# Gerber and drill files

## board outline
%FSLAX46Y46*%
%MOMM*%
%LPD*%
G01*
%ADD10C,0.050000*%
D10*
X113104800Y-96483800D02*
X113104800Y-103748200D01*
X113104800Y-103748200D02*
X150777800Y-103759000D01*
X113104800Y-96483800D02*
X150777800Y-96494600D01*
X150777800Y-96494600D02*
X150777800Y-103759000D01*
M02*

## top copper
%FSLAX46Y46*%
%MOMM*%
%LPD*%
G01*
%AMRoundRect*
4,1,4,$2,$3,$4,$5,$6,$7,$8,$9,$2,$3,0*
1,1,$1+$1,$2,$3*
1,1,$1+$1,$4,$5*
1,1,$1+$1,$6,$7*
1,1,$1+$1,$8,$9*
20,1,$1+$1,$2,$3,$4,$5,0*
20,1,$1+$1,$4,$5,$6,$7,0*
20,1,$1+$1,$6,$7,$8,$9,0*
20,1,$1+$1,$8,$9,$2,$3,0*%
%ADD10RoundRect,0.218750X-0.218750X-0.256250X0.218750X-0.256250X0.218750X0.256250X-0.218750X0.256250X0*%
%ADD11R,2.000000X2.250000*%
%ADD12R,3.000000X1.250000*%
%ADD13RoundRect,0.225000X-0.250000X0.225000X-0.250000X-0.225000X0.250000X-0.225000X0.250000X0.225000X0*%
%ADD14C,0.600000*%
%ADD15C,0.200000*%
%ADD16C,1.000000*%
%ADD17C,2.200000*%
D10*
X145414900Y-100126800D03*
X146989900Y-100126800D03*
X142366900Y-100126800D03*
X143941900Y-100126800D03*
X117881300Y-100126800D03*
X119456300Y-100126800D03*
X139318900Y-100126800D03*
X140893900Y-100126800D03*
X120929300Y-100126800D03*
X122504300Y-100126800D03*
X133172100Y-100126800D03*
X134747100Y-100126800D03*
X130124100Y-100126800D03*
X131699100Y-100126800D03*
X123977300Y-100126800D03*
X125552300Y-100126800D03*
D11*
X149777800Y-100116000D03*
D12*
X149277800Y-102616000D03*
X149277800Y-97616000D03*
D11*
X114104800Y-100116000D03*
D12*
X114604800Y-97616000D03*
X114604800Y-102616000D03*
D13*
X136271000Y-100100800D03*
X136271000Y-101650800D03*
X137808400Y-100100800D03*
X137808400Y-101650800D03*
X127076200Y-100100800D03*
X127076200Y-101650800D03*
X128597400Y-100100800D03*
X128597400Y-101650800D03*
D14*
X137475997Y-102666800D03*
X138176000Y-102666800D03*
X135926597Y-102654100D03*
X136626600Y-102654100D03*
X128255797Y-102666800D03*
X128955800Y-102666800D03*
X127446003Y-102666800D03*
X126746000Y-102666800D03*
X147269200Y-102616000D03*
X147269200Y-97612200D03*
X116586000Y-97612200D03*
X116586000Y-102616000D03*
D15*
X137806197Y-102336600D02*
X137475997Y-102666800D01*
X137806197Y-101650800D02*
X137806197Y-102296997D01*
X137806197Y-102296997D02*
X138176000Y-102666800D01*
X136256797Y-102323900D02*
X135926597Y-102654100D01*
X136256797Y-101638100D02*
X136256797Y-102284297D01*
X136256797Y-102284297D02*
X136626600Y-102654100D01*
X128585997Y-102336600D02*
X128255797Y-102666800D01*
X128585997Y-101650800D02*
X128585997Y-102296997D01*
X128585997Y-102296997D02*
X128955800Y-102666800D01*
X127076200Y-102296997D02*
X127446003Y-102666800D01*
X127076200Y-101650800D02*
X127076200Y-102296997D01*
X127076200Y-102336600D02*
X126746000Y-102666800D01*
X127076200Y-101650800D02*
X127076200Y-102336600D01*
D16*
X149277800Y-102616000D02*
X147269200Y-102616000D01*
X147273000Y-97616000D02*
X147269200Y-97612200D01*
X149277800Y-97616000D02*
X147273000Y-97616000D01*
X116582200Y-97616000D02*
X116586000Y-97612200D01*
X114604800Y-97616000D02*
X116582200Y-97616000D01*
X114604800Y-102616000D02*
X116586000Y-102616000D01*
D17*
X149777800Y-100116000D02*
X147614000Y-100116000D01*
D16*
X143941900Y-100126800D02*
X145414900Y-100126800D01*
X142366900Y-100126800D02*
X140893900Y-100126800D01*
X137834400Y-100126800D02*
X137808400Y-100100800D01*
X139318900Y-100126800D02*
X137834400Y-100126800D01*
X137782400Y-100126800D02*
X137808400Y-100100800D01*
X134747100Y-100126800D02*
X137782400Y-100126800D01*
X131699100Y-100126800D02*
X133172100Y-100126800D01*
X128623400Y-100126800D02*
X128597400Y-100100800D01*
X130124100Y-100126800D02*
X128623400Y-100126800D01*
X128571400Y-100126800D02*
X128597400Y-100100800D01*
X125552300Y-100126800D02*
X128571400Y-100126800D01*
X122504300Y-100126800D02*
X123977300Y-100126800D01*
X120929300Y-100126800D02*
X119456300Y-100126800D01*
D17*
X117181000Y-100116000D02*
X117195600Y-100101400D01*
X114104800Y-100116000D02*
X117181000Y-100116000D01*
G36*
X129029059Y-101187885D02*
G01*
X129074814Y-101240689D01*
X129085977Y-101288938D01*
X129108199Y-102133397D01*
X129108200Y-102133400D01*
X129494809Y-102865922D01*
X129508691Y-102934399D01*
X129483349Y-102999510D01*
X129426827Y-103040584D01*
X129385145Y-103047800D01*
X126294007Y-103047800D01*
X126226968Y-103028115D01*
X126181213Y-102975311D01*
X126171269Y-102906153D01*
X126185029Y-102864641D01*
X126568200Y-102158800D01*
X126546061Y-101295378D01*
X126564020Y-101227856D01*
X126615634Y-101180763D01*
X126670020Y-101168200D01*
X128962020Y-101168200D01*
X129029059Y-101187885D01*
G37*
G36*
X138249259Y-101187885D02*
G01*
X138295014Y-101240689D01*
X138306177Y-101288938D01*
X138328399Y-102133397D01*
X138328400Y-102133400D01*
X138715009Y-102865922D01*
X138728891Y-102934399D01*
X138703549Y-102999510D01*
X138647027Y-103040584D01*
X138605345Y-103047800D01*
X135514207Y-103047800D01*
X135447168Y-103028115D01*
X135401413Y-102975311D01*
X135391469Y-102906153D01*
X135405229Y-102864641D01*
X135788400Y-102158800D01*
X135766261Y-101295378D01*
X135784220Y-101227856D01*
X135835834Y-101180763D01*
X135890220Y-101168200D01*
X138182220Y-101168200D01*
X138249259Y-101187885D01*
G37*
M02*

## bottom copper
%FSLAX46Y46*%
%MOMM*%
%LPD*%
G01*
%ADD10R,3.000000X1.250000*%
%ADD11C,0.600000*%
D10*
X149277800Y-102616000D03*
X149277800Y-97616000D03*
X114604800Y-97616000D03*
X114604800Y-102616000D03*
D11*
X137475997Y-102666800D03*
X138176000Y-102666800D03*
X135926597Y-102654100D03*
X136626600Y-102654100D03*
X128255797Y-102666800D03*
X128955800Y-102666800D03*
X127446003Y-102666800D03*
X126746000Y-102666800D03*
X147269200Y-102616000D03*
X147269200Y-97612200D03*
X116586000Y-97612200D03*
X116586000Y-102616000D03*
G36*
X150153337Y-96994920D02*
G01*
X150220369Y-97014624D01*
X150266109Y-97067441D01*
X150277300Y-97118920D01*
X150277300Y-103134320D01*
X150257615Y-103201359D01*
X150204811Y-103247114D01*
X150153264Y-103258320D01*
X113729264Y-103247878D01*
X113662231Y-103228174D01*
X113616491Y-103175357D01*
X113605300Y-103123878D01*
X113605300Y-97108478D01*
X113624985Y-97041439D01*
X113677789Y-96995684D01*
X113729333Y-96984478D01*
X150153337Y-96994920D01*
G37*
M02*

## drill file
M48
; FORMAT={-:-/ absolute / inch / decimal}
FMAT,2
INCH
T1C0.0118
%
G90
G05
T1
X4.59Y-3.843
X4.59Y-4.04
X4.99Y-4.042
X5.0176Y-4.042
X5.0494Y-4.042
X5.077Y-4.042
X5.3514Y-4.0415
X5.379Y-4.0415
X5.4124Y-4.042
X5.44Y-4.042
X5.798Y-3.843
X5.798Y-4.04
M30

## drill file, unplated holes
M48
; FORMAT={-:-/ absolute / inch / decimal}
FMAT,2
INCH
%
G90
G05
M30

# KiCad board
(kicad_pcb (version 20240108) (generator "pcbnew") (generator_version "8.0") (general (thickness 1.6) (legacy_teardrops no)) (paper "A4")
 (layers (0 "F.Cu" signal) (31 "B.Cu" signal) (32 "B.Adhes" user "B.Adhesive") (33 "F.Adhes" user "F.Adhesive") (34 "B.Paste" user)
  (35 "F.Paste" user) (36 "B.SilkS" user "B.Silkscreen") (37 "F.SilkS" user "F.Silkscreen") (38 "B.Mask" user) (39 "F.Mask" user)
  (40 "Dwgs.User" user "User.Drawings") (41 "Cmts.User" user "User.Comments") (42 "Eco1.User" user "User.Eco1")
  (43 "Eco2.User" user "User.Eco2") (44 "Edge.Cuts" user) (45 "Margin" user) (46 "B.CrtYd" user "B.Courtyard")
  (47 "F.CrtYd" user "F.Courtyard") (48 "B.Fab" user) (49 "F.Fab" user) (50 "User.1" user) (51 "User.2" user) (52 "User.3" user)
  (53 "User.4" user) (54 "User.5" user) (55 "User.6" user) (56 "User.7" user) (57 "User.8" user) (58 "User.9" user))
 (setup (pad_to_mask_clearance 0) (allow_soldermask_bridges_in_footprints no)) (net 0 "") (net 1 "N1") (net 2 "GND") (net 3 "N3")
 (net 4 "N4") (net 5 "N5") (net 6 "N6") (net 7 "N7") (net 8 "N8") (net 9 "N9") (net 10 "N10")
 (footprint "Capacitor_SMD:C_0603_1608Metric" (layer "F.Cu") (at 128.5974 100.8758 -90)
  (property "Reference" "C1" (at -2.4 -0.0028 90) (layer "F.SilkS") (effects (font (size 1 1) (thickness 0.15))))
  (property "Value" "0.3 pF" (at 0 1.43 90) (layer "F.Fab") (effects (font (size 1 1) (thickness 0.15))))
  (pad "1" smd roundrect (at -0.775 0 270) (size 0.9 0.95) (layers "F.Cu" "F.Paste" "F.Mask") (roundrect_rratio 0.25) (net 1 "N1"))
  (pad "2" smd roundrect (at 0.775 0 270) (size 0.9 0.95) (layers "F.Cu" "F.Paste" "F.Mask") (roundrect_rratio 0.25) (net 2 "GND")))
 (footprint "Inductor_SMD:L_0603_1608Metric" (layer "F.Cu") (at 133.9596 100.1268)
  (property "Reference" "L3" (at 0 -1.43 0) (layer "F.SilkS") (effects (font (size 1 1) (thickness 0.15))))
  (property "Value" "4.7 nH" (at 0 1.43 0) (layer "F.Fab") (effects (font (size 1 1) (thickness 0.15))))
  (pad "1" smd roundrect (at -0.7875 0) (size 0.875 0.95) (layers "F.Cu" "F.Paste" "F.Mask") (roundrect_rratio 0.25) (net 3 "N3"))
  (pad "2" smd roundrect (at 0.7875 0) (size 0.875 0.95) (layers "F.Cu" "F.Paste" "F.Mask") (roundrect_rratio 0.25) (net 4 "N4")))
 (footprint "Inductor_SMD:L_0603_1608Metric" (layer "F.Cu") (at 146.2024 100.1268)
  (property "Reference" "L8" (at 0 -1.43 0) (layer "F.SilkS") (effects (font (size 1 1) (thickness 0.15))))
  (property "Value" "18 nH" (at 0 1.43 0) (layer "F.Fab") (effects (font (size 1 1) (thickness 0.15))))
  (pad "1" smd roundrect (at -0.7875 0) (size 0.875 0.95) (layers "F.Cu" "F.Paste" "F.Mask") (roundrect_rratio 0.25) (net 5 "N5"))
  (pad "2" smd roundrect (at 0.7875 0) (size 0.875 0.95) (layers "F.Cu" "F.Paste" "F.Mask") (roundrect_rratio 0.25) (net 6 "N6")))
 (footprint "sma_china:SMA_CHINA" (layer "F.Cu") (at 150.7778 100.116 90)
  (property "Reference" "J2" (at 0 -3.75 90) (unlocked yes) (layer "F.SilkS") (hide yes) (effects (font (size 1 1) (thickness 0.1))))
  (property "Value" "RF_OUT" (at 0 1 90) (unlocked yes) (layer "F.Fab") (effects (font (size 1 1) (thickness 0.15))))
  (pad "1" smd rect (at 0 -1 90) (size 2.25 2) (layers "F.Cu" "F.Paste" "F.Mask") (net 6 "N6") (thermal_bridge_angle 45))
  (pad "2" smd rect (at -2.5 -1.5 90) (size 1.25 3) (layers "F.Cu" "F.Paste" "F.Mask") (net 2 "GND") (thermal_bridge_angle 45))
  (pad "2" smd rect (at -2.5 -1.5 90) (size 1.25 3) (layers "B.Cu" "B.Paste" "B.Mask") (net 2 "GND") (thermal_bridge_angle 45))
  (pad "2" smd rect (at 2.5 -1.5 90) (size 1.25 3) (layers "F.Cu" "F.Paste" "F.Mask") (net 2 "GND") (thermal_bridge_angle 45))
  (pad "2" smd rect (at 2.5 -1.5 90) (size 1.25 3) (layers "B.Cu" "B.Paste" "B.Mask") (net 2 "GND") (thermal_bridge_angle 45)))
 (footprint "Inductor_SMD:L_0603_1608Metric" (layer "F.Cu") (at 121.7168 100.1268)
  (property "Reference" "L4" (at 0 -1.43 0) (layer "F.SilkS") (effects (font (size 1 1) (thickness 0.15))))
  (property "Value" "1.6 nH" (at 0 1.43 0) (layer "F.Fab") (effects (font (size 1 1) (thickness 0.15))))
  (pad "1" smd roundrect (at -0.7875 0) (size 0.875 0.95) (layers "F.Cu" "F.Paste" "F.Mask") (roundrect_rratio 0.25) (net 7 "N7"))
  (pad "2" smd roundrect (at 0.7875 0) (size 0.875 0.95) (layers "F.Cu" "F.Paste" "F.Mask") (roundrect_rratio 0.25) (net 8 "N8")))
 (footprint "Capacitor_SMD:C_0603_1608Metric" (layer "F.Cu") (at 137.8084 100.8758 -90)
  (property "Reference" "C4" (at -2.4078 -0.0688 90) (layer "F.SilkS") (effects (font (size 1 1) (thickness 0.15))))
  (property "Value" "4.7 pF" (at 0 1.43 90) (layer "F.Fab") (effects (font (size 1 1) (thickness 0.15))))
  (pad "1" smd roundrect (at -0.775 0 270) (size 0.9 0.95) (layers "F.Cu" "F.Paste" "F.Mask") (roundrect_rratio 0.25) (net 4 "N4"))
  (pad "2" smd roundrect (at 0.775 0 270) (size 0.9 0.95) (layers "F.Cu" "F.Paste" "F.Mask") (roundrect_rratio 0.25) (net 2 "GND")))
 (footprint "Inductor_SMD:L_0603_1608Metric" (layer "F.Cu") (at 124.7648 100.1268)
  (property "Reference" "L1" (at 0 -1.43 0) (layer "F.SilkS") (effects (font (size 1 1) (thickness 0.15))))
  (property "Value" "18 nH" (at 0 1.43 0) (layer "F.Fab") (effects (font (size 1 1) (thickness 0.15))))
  (pad "1" smd roundrect (at -0.7875 0) (size 0.875 0.95) (layers "F.Cu" "F.Paste" "F.Mask") (roundrect_rratio 0.25) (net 8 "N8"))
  (pad "2" smd roundrect (at 0.7875 0) (size 0.875 0.95) (layers "F.Cu" "F.Paste" "F.Mask") (roundrect_rratio 0.25) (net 1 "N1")))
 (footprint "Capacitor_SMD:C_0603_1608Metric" (layer "F.Cu") (at 127.0762 100.8758 -90)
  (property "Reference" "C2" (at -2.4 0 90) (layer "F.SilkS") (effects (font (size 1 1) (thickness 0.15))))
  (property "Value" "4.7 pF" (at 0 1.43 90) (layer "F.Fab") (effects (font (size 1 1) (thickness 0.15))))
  (pad "1" smd roundrect (at -0.775 0 270) (size 0.9 0.95) (layers "F.Cu" "F.Paste" "F.Mask") (roundrect_rratio 0.25) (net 1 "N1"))
  (pad "2" smd roundrect (at 0.775 0 270) (size 0.9 0.95) (layers "F.Cu" "F.Paste" "F.Mask") (roundrect_rratio 0.25) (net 2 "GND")))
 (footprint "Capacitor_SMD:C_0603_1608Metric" (layer "F.Cu") (at 136.271 100.8758 -90)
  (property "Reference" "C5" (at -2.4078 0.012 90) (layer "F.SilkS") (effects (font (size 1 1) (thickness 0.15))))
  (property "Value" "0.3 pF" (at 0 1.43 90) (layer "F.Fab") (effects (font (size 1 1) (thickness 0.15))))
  (pad "1" smd roundrect (at -0.775 0 270) (size 0.9 0.95) (layers "F.Cu" "F.Paste" "F.Mask") (roundrect_rratio 0.25) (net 4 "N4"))
  (pad "2" smd roundrect (at 0.775 0 270) (size 0.9 0.95) (layers "F.Cu" "F.Paste" "F.Mask") (roundrect_rratio 0.25) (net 2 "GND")))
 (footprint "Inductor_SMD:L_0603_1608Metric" (layer "F.Cu") (at 130.9116 100.1268)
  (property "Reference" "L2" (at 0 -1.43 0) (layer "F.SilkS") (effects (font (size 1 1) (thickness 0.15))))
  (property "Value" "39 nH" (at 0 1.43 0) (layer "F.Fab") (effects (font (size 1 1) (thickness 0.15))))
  (pad "1" smd roundrect (at -0.7875 0) (size 0.875 0.95) (layers "F.Cu" "F.Paste" "F.Mask") (roundrect_rratio 0.25) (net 1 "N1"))
  (pad "2" smd roundrect (at 0.7875 0) (size 0.875 0.95) (layers "F.Cu" "F.Paste" "F.Mask") (roundrect_rratio 0.25) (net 3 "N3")))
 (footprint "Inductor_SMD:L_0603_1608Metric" (layer "F.Cu") (at 140.1064 100.1268)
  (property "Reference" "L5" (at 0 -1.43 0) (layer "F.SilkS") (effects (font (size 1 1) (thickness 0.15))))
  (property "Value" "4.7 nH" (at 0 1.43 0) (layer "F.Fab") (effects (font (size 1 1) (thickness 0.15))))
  (pad "1" smd roundrect (at -0.7875 0) (size 0.875 0.95) (layers "F.Cu" "F.Paste" "F.Mask") (roundrect_rratio 0.25) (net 4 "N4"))
  (pad "2" smd roundrect (at 0.7875 0) (size 0.875 0.95) (layers "F.Cu" "F.Paste" "F.Mask") (roundrect_rratio 0.25) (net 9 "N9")))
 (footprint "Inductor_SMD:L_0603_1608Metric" (layer "F.Cu") (at 143.1544 100.1268)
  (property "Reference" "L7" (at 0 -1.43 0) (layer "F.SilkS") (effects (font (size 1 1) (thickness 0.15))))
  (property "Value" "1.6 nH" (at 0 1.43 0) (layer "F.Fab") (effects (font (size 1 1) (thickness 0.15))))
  (pad "1" smd roundrect (at -0.7875 0) (size 0.875 0.95) (layers "F.Cu" "F.Paste" "F.Mask") (roundrect_rratio 0.25) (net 9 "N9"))
  (pad "2" smd roundrect (at 0.7875 0) (size 0.875 0.95) (layers "F.Cu" "F.Paste" "F.Mask") (roundrect_rratio 0.25) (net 5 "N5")))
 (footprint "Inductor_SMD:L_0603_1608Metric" (layer "F.Cu") (at 118.6688 100.1268)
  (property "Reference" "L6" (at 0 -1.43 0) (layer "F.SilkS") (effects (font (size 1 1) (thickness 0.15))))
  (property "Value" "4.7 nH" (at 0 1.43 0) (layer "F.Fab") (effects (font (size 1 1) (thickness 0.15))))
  (pad "1" smd roundrect (at -0.7875 0) (size 0.875 0.95) (layers "F.Cu" "F.Paste" "F.Mask") (roundrect_rratio 0.25) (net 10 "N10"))
  (pad "2" smd roundrect (at 0.7875 0) (size 0.875 0.95) (layers "F.Cu" "F.Paste" "F.Mask") (roundrect_rratio 0.25) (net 7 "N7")))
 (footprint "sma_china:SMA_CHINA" (layer "F.Cu") (at 113.1048 100.116 -90)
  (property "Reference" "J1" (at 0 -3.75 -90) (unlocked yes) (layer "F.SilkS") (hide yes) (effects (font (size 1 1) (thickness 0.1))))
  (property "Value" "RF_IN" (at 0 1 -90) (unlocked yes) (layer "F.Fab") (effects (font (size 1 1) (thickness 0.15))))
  (pad "1" smd rect (at 0 -1 270) (size 2.25 2) (layers "F.Cu" "F.Paste" "F.Mask") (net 10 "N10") (thermal_bridge_angle 45))
  (pad "2" smd rect (at -2.5 -1.5 270) (size 1.25 3) (layers "F.Cu" "F.Paste" "F.Mask") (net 2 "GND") (thermal_bridge_angle 45))
  (pad "2" smd rect (at -2.5 -1.5 270) (size 1.25 3) (layers "B.Cu" "B.Paste" "B.Mask") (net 2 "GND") (thermal_bridge_angle 45))
  (pad "2" smd rect (at 2.5 -1.5 270) (size 1.25 3) (layers "F.Cu" "F.Paste" "F.Mask") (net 2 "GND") (thermal_bridge_angle 45))
  (pad "2" smd rect (at 2.5 -1.5 270) (size 1.25 3) (layers "B.Cu" "B.Paste" "B.Mask") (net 2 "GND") (thermal_bridge_angle 45)))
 (gr_line (start 150.7778 96.4946) (end 150.7778 103.759) (stroke (width 0.05) (type default)) (layer "Edge.Cuts"))
 (gr_line (start 113.1048 96.4838) (end 150.7778 96.4946) (stroke (width 0.05) (type default)) (layer "Edge.Cuts"))
 (gr_line (start 113.1048 96.4838) (end 113.1048 103.7482) (stroke (width 0.05) (type default)) (layer "Edge.Cuts"))
 (gr_line (start 113.1048 103.7482) (end 150.7778 103.759) (stroke (width 0.05) (type default)) (layer "Edge.Cuts"))
 (segment (start 147.273 97.616) (end 147.2692 97.6122) (width 1) (layer "F.Cu") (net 2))
 (segment (start 136.256797 101.6381) (end 136.256797 102.284297) (width 0.2) (layer "F.Cu") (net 2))
 (segment (start 127.0762 102.296997) (end 127.446003 102.6668) (width 0.2) (layer "F.Cu") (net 2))
 (segment (start 137.806197 101.6508) (end 137.806197 102.296997) (width 0.2) (layer "F.Cu") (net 2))
 (segment (start 127.0762 101.6508) (end 127.0762 102.296997) (width 0.2) (layer "F.Cu") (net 2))
 (segment (start 137.806197 102.3366) (end 137.475997 102.6668) (width 0.2) (layer "F.Cu") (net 2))
 (segment (start 127.0762 101.6508) (end 127.0762 102.3366) (width 0.2) (layer "F.Cu") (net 2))
 (segment (start 114.6048 102.616) (end 116.586 102.616) (width 1) (layer "F.Cu") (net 2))
 (segment (start 149.2778 97.616) (end 147.273 97.616) (width 1) (layer "F.Cu") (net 2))
 (segment (start 128.585997 101.6508) (end 128.585997 102.296997) (width 0.2) (layer "F.Cu") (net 2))
 (segment (start 128.585997 102.3366) (end 128.255797 102.6668) (width 0.2) (layer "F.Cu") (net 2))
 (segment (start 127.0762 102.3366) (end 126.746 102.6668) (width 0.2) (layer "F.Cu") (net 2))
 (segment (start 149.2778 102.616) (end 147.2692 102.616) (width 1) (layer "F.Cu") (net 2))
 (segment (start 136.256797 102.284297) (end 136.6266 102.6541) (width 0.2) (layer "F.Cu") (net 2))
 (segment (start 128.585997 102.296997) (end 128.9558 102.6668) (width 0.2) (layer "F.Cu") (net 2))
 (segment (start 136.256797 102.3239) (end 135.926597 102.6541) (width 0.2) (layer "F.Cu") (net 2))
 (segment (start 137.806197 102.296997) (end 138.176 102.6668) (width 0.2) (layer "F.Cu") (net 2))
 (segment (start 114.6048 97.616) (end 116.5822 97.616) (width 1) (layer "F.Cu") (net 2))
 (segment (start 116.5822 97.616) (end 116.586 97.6122) (width 1) (layer "F.Cu") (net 2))
 (via (at 136.6266 102.6541) (size 0.6) (drill 0.3) (layers "F.Cu" "B.Cu") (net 2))
 (via (at 138.176 102.6668) (size 0.6) (drill 0.3) (layers "F.Cu" "B.Cu") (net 2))
 (via (at 135.926597 102.6541) (size 0.6) (drill 0.3) (layers "F.Cu" "B.Cu") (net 2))
 (via (at 126.746 102.6668) (size 0.6) (drill 0.3) (layers "F.Cu" "B.Cu") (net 2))
 (via (at 137.475997 102.6668) (size 0.6) (drill 0.3) (layers "F.Cu" "B.Cu") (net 2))
 (via (at 127.446003 102.6668) (size 0.6) (drill 0.3) (layers "F.Cu" "B.Cu") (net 2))
 (via (at 116.586 102.616) (size 0.6) (drill 0.3) (layers "F.Cu" "B.Cu") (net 2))
 (via (at 128.255797 102.6668) (size 0.6) (drill 0.3) (layers "F.Cu" "B.Cu") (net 2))
 (via (at 116.586 97.6122) (size 0.6) (drill 0.3) (layers "F.Cu" "B.Cu") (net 2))
 (via (at 128.9558 102.6668) (size 0.6) (drill 0.3) (layers "F.Cu" "B.Cu") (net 2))
 (via (at 147.2692 97.6122) (size 0.6) (drill 0.3) (layers "F.Cu" "B.Cu") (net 2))
 (via (at 147.2692 102.616) (size 0.6) (drill 0.3) (layers "F.Cu" "B.Cu") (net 2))
 (segment (start 128.6234 100.1268) (end 128.5974 100.1008) (width 1) (layer "F.Cu") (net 1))
 (segment (start 130.1241 100.1268) (end 128.6234 100.1268) (width 1) (layer "F.Cu") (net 1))
 (segment (start 125.5523 100.1268) (end 128.5714 100.1268) (width 1) (layer "F.Cu") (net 1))
 (segment (start 128.5714 100.1268) (end 128.5974 100.1008) (width 1) (layer "F.Cu") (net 1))
 (segment (start 134.7471 100.1268) (end 137.7824 100.1268) (width 1) (layer "F.Cu") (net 4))
 (segment (start 137.7824 100.1268) (end 137.8084 100.1008) (width 1) (layer "F.Cu") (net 4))
 (segment (start 137.8344 100.1268) (end 137.8084 100.1008) (width 1) (layer "F.Cu") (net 4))
 (segment (start 139.3189 100.1268) (end 137.8344 100.1268) (width 1) (layer "F.Cu") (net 4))
 (segment (start 114.1048 100.116) (end 117.181 100.116) (width 2.2) (layer "F.Cu") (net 10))
 (segment (start 117.181 100.116) (end 117.1956 100.1014) (width 2.2) (layer "F.Cu") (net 10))
 (segment (start 149.7778 100.116) (end 147.614 100.116) (width 2.2) (layer "F.Cu") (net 6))
 (segment (start 122.5043 100.1268) (end 123.9773 100.1268) (width 1) (layer "F.Cu") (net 8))
 (segment (start 131.6991 100.1268) (end 133.1721 100.1268) (width 1) (layer "F.Cu") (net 3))
 (segment (start 120.9293 100.1268) (end 119.4563 100.1268) (width 1) (layer "F.Cu") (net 7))
 (segment (start 142.3669 100.1268) (end 140.8939 100.1268) (width 1) (layer "F.Cu") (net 9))
 (segment (start 143.9419 100.1268) (end 145.4149 100.1268) (width 1) (layer "F.Cu") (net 5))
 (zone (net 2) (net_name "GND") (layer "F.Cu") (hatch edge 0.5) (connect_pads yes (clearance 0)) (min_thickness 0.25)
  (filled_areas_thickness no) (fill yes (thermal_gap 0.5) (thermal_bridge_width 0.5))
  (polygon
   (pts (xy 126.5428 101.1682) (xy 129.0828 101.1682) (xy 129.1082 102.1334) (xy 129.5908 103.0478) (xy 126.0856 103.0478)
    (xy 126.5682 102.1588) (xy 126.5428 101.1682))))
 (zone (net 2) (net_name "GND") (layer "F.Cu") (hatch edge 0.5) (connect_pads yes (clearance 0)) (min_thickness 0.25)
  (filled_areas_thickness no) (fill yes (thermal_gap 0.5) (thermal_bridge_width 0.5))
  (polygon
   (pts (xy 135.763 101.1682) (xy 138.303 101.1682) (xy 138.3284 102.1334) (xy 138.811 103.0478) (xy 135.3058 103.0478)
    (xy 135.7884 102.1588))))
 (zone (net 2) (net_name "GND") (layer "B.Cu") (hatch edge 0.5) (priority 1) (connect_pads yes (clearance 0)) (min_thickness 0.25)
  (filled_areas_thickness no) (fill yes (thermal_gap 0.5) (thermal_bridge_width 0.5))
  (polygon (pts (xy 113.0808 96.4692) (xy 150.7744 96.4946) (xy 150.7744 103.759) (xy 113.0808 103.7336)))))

